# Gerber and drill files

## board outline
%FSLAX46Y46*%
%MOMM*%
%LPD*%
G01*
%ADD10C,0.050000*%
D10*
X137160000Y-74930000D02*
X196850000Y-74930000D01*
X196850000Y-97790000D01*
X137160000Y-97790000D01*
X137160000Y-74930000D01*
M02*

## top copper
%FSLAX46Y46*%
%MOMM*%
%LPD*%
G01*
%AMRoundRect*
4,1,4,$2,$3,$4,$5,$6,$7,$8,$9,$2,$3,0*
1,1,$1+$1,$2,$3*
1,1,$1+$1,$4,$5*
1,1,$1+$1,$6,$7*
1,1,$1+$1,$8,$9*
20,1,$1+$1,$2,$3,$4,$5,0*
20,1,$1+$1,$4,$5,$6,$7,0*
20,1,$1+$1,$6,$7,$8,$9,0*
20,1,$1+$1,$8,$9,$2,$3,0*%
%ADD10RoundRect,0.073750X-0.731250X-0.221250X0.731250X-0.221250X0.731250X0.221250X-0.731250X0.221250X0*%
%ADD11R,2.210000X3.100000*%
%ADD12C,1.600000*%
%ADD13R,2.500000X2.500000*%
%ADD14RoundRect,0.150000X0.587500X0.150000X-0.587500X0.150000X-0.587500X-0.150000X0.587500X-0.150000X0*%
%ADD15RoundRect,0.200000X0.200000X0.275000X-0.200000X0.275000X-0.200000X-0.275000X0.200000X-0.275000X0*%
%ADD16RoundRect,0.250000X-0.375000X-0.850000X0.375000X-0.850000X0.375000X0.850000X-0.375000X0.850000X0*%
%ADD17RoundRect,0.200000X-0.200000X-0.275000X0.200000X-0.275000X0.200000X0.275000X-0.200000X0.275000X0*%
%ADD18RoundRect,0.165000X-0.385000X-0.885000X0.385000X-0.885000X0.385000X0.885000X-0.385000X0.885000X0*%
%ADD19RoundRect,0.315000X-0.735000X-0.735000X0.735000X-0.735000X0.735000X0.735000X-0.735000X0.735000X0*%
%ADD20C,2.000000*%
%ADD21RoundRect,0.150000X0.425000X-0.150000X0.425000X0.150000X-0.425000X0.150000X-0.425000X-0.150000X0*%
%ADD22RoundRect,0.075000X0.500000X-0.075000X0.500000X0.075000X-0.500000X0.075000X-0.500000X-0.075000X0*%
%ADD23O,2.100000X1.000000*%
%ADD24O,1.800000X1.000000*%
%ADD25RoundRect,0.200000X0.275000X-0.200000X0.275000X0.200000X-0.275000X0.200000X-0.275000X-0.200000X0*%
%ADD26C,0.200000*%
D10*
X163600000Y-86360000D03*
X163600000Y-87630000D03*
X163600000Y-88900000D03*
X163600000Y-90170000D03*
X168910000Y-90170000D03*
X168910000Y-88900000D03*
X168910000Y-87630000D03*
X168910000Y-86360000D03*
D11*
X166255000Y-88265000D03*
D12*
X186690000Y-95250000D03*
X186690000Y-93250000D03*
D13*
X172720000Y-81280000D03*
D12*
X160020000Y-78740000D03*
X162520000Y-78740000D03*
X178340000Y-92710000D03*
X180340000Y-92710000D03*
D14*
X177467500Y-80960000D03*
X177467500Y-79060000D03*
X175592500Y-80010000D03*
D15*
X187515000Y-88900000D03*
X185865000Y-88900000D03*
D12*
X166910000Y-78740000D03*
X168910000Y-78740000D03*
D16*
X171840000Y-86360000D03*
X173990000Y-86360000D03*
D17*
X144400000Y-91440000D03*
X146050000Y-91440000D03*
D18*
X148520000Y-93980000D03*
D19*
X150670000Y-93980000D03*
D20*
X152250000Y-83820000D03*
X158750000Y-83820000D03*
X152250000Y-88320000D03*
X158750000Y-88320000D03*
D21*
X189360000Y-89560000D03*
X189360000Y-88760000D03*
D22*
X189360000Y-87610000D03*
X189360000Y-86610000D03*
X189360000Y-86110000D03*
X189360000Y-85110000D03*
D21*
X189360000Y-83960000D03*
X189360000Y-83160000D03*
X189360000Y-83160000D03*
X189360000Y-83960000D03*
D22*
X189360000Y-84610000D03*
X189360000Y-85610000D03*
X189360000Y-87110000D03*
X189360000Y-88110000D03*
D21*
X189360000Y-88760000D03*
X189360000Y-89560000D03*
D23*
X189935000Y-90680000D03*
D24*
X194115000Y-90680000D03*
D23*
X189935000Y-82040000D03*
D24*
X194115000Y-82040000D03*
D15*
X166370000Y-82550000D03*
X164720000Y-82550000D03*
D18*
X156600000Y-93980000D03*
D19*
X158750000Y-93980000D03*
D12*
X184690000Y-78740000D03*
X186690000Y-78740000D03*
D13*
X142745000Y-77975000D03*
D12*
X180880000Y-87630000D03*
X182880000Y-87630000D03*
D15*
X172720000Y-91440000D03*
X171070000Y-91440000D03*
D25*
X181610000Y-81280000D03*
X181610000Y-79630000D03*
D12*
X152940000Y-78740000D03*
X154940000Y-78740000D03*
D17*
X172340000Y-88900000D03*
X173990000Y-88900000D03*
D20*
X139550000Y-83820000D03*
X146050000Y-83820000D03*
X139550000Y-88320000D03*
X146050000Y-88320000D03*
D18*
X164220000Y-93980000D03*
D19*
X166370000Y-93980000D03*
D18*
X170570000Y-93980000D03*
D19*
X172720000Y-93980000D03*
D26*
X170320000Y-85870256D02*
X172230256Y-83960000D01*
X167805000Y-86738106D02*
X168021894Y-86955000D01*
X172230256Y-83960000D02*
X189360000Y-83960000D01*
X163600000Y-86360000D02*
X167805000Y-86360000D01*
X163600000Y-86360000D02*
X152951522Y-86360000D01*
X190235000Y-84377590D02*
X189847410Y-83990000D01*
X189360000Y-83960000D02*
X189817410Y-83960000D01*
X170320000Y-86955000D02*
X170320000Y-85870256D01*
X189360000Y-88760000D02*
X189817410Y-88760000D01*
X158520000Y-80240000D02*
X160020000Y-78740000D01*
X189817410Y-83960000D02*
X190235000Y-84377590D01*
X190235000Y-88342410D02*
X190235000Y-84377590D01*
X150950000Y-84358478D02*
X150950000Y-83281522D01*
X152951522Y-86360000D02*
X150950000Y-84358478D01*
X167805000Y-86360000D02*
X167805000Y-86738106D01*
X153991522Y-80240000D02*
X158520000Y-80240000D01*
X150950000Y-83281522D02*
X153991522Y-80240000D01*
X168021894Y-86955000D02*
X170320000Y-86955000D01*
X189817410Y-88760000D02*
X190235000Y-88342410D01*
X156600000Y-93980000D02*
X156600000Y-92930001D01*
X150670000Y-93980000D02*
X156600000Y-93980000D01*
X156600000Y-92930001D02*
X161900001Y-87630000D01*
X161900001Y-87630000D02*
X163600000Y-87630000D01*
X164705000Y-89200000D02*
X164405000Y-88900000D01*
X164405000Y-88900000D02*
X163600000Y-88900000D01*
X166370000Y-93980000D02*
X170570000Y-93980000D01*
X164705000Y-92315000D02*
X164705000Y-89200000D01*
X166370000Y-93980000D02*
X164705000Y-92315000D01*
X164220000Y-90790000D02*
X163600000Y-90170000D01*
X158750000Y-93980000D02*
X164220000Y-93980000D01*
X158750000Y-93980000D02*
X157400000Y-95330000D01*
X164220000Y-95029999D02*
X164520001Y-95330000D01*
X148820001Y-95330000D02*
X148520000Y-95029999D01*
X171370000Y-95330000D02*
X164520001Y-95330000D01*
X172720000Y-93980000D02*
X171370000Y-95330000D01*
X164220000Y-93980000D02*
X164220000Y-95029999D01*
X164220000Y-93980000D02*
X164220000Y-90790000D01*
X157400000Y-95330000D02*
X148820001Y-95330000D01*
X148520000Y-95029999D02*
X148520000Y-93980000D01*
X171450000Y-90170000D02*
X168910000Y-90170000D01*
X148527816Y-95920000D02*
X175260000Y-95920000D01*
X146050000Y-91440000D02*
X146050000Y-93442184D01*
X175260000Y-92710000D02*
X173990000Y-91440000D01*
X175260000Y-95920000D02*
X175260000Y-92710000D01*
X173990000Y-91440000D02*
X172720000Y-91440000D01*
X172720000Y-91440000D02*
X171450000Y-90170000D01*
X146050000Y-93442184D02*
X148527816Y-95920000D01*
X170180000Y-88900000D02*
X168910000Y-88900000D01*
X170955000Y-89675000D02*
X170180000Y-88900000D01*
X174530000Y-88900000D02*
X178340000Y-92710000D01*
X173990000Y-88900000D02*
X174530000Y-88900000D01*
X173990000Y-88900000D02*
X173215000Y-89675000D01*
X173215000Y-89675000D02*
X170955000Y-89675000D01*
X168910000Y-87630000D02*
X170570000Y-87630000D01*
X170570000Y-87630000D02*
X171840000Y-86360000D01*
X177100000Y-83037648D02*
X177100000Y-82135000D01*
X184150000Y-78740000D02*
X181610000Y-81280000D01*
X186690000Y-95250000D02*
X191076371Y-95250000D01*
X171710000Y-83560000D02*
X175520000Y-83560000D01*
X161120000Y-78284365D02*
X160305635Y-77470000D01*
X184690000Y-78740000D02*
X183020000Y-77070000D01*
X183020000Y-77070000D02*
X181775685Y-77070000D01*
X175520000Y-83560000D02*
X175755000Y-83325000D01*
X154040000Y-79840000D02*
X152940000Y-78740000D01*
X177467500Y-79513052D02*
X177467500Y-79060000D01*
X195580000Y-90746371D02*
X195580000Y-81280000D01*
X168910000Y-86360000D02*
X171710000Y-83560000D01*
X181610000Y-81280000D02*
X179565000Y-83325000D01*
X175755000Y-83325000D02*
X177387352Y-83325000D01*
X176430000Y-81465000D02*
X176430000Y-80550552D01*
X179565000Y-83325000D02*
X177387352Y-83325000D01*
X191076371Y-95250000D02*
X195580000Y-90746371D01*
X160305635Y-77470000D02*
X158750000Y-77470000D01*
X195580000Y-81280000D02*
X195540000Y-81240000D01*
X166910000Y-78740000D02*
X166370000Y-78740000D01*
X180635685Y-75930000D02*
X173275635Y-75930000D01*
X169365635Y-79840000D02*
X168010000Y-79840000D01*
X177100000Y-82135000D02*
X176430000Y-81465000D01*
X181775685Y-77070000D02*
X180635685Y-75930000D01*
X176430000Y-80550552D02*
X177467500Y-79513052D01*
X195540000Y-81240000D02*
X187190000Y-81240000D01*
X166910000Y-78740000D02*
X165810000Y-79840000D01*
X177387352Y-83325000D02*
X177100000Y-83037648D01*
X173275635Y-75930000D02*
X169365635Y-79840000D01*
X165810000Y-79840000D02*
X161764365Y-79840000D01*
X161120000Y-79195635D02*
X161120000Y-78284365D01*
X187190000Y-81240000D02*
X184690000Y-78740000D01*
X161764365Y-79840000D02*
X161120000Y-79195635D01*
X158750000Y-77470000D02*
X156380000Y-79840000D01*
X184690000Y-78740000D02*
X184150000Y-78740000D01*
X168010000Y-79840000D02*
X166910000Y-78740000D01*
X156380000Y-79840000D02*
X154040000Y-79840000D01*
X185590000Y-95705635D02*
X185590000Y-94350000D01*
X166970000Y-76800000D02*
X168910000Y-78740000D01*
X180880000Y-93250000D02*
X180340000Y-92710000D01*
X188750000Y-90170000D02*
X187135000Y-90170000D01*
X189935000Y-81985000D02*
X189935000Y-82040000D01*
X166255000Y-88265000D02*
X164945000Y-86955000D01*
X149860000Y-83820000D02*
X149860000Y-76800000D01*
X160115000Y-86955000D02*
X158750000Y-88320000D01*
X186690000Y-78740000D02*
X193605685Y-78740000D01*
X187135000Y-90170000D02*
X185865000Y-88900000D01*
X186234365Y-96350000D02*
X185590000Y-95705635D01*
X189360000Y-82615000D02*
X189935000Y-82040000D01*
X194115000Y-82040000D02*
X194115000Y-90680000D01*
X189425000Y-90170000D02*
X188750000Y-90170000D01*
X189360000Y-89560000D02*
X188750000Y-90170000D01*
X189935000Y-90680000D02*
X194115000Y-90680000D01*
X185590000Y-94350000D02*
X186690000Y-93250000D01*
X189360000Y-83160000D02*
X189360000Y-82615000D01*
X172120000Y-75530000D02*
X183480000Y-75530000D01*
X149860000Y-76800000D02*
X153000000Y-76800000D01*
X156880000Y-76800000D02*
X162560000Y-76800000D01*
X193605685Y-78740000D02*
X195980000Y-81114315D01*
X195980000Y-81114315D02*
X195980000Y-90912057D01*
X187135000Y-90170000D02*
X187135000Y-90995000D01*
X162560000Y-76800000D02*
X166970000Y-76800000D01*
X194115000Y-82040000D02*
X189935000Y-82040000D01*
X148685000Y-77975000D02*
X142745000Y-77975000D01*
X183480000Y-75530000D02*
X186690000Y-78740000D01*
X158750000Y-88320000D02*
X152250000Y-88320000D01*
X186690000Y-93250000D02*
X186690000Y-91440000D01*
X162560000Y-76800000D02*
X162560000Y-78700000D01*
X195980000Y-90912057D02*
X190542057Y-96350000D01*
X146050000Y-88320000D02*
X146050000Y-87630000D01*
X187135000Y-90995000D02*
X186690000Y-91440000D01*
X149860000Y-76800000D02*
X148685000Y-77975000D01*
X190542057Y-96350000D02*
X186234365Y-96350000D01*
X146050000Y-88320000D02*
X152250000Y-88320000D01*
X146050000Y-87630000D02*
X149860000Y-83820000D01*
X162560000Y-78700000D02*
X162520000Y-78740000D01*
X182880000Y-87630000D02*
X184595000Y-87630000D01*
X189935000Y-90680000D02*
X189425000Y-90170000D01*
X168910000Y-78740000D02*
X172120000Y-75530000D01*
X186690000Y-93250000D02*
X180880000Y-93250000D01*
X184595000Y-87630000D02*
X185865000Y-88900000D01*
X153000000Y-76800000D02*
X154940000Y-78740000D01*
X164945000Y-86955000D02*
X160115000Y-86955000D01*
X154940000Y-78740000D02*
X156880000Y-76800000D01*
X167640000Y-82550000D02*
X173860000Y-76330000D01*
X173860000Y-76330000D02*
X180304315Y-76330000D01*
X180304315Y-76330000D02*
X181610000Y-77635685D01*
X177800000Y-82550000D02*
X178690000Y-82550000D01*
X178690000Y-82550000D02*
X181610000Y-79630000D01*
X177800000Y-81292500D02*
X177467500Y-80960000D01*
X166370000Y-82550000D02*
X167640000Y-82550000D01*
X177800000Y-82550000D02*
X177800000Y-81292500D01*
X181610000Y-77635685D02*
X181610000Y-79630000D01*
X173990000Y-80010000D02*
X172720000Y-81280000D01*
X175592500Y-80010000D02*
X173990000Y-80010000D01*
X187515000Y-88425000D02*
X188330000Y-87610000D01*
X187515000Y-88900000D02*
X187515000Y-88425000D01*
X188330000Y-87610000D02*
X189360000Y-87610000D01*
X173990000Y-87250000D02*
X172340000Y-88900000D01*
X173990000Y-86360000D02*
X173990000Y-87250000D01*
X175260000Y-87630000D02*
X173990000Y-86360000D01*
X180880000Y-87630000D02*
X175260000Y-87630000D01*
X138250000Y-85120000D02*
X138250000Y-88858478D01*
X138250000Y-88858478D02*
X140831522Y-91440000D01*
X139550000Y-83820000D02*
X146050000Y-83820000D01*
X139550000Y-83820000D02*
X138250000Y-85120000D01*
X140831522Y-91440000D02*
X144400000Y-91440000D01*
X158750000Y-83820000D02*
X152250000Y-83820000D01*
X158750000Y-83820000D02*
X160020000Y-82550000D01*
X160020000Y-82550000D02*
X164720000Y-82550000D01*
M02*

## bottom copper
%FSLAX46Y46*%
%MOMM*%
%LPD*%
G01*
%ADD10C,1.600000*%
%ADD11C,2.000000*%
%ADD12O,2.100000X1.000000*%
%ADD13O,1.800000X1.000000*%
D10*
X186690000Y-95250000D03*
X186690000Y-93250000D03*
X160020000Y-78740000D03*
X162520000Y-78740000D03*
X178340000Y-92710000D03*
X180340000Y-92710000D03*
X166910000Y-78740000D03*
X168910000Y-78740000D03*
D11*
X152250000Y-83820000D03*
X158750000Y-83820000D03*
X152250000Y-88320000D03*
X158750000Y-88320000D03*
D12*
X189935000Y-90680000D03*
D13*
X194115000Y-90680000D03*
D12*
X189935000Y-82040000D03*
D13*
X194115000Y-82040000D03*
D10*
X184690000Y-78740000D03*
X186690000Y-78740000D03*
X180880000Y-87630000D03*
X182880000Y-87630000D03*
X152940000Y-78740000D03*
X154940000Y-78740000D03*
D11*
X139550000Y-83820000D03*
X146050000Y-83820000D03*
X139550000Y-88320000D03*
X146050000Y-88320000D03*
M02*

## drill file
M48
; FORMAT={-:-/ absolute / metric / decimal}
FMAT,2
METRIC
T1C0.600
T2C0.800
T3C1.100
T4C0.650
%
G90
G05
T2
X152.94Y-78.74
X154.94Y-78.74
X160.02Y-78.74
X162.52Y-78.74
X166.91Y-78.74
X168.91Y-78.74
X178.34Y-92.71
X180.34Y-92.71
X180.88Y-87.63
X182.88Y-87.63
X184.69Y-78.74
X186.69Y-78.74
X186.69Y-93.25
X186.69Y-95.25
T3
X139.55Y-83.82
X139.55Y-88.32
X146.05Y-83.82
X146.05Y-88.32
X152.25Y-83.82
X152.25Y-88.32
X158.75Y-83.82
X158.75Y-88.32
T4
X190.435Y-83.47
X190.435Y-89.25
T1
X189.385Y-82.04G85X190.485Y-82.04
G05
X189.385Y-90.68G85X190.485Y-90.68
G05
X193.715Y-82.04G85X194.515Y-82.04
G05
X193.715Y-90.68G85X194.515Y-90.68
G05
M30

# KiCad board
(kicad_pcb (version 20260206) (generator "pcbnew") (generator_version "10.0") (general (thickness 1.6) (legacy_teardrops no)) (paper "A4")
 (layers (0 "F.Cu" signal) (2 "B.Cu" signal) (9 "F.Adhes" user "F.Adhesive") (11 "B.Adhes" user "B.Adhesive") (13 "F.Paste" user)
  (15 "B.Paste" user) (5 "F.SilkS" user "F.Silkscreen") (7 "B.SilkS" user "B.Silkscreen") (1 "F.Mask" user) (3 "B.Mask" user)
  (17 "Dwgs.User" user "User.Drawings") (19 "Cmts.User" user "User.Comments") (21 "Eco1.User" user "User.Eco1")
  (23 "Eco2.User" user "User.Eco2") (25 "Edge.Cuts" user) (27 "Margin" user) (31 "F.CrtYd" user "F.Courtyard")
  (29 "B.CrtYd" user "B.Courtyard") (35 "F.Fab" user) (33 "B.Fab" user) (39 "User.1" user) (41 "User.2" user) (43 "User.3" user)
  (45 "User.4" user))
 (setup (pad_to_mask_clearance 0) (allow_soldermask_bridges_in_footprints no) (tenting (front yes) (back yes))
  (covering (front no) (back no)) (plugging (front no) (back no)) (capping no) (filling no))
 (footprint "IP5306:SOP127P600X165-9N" (layer "F.Cu") (at 166.255 88.265)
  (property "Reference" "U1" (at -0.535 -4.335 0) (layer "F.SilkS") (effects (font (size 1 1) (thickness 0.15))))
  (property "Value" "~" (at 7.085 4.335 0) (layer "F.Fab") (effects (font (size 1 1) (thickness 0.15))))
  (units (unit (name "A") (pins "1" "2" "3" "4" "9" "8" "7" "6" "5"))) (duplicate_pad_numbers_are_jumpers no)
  (pad "1" smd roundrect (at -2.655 -1.905) (size 1.61 0.59) (layers "F.Cu" "F.Mask" "F.Paste") (roundrect_rratio 0.125)
   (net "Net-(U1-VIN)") (solder_mask_margin 0.102))
  (pad "2" smd roundrect (at -2.655 -0.635) (size 1.61 0.59) (layers "F.Cu" "F.Mask" "F.Paste") (roundrect_rratio 0.125) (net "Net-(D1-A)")
   (solder_mask_margin 0.102))
  (pad "3" smd roundrect (at -2.655 0.635) (size 1.61 0.59) (layers "F.Cu" "F.Mask" "F.Paste") (roundrect_rratio 0.125) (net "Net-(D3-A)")
   (solder_mask_margin 0.102))
  (pad "4" smd roundrect (at -2.655 1.905) (size 1.61 0.59) (layers "F.Cu" "F.Mask" "F.Paste") (roundrect_rratio 0.125) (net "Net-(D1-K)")
   (solder_mask_margin 0.102))
  (pad "5" smd roundrect (at 2.655 1.905) (size 1.61 0.59) (layers "F.Cu" "F.Mask" "F.Paste") (roundrect_rratio 0.125) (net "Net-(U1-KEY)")
   (solder_mask_margin 0.102))
  (pad "6" smd roundrect (at 2.655 0.635) (size 1.61 0.59) (layers "F.Cu" "F.Mask" "F.Paste") (roundrect_rratio 0.125) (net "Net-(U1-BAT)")
   (solder_mask_margin 0.102))
  (pad "7" smd roundrect (at 2.655 -0.635) (size 1.61 0.59) (layers "F.Cu" "F.Mask" "F.Paste") (roundrect_rratio 0.125) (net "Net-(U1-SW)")
   (solder_mask_margin 0.102))
  (pad "8" smd roundrect (at 2.655 -1.905) (size 1.61 0.59) (layers "F.Cu" "F.Mask" "F.Paste") (roundrect_rratio 0.125) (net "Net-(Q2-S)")
   (solder_mask_margin 0.102))
  (pad "9" smd rect (at 0 0) (size 2.21 3.1) (layers "F.Cu" "F.Mask") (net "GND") (solder_mask_margin 0.102)))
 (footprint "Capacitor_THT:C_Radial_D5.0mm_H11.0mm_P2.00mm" (layer "F.Cu") (at 186.69 95.25 90)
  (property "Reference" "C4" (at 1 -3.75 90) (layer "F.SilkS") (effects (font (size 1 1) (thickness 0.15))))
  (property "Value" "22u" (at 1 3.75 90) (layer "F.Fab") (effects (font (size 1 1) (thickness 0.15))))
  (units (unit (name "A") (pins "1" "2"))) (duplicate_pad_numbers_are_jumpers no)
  (pad "1" thru_hole circle (at 0 0 90) (size 1.6 1.6) (drill 0.8) (layers "*.Cu" "*.Mask") (remove_unused_layers no) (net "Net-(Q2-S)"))
  (pad "2" thru_hole circle (at 2 0 90) (size 1.6 1.6) (drill 0.8) (layers "*.Cu" "*.Mask") (remove_unused_layers no) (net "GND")))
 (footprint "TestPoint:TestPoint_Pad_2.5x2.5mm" (layer "F.Cu") (at 172.72 81.28)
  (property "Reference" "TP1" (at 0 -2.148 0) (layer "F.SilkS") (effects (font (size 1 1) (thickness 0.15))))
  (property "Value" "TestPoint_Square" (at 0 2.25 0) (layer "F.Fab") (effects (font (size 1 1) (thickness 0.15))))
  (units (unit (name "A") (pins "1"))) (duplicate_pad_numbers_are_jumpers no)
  (pad "1" smd rect (at 0 0) (size 2.5 2.5) (layers "F.Cu" "F.Mask") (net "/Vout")))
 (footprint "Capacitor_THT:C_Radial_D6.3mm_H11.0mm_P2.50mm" (layer "F.Cu") (at 160.02 78.74)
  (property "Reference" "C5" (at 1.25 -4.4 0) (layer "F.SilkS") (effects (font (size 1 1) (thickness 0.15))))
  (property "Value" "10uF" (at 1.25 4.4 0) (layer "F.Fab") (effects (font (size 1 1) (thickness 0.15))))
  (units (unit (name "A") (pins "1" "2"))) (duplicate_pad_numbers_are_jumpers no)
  (pad "1" thru_hole circle (at 0 0) (size 1.6 1.6) (drill 0.8) (layers "*.Cu" "*.Mask") (remove_unused_layers no) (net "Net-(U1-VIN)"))
  (pad "2" thru_hole circle (at 2.5 0) (size 1.6 1.6) (drill 0.8) (layers "*.Cu" "*.Mask") (remove_unused_layers no) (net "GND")))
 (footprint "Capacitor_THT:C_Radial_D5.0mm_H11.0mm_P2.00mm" (layer "F.Cu") (at 178.34 92.71)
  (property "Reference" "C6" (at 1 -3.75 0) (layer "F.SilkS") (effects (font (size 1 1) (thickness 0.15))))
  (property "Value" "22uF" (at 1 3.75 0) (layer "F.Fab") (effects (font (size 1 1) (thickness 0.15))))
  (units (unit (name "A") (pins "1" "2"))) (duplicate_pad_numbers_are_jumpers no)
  (pad "1" thru_hole circle (at 0 0) (size 1.6 1.6) (drill 0.8) (layers "*.Cu" "*.Mask") (remove_unused_layers no) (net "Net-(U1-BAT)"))
  (pad "2" thru_hole circle (at 2 0) (size 1.6 1.6) (drill 0.8) (layers "*.Cu" "*.Mask") (remove_unused_layers no) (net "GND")))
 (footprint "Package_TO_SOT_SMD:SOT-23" (layer "F.Cu") (at 176.53 80.01 180)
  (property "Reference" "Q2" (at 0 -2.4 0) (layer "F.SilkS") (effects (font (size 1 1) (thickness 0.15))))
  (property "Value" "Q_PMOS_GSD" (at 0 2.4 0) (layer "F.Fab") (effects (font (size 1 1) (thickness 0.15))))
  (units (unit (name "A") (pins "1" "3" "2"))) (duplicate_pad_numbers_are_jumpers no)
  (pad "1" smd roundrect (at -0.9375 -0.95 180) (size 1.475 0.6) (layers "F.Cu" "F.Mask" "F.Paste") (roundrect_rratio 0.25)
   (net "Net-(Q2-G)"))
  (pad "2" smd roundrect (at -0.9375 0.95 180) (size 1.475 0.6) (layers "F.Cu" "F.Mask" "F.Paste") (roundrect_rratio 0.25)
   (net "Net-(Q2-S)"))
  (pad "3" smd roundrect (at 0.9375 0 180) (size 1.475 0.6) (layers "F.Cu" "F.Mask" "F.Paste") (roundrect_rratio 0.25) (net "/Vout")))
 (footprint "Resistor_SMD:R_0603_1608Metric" (layer "F.Cu") (at 186.69 88.9 180)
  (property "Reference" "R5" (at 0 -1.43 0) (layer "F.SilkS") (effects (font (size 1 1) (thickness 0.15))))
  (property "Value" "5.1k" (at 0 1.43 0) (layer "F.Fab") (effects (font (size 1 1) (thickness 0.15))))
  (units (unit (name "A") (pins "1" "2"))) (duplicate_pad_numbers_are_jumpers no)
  (pad "1" smd roundrect (at -0.825 0 180) (size 0.8 0.95) (layers "F.Cu" "F.Mask" "F.Paste") (roundrect_rratio 0.25) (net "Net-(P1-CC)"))
  (pad "2" smd roundrect (at 0.825 0 180) (size 0.8 0.95) (layers "F.Cu" "F.Mask" "F.Paste") (roundrect_rratio 0.25) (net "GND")))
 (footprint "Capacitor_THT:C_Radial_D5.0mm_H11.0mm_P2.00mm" (layer "F.Cu") (at 166.91 78.74)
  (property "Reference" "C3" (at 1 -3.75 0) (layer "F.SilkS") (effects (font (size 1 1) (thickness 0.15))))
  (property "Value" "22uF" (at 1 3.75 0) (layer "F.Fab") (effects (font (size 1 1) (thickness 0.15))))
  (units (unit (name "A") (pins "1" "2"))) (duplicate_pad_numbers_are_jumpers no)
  (pad "1" thru_hole circle (at 0 0) (size 1.6 1.6) (drill 0.8) (layers "*.Cu" "*.Mask") (remove_unused_layers no) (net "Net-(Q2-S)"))
  (pad "2" thru_hole circle (at 2 0) (size 1.6 1.6) (drill 0.8) (layers "*.Cu" "*.Mask") (remove_unused_layers no) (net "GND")))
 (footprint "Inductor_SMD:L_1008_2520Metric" (layer "F.Cu") (at 172.915 86.36)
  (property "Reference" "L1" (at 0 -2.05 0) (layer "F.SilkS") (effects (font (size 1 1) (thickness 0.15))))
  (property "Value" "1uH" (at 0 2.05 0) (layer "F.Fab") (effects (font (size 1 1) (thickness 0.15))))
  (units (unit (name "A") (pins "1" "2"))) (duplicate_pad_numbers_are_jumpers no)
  (pad "1" smd roundrect (at -1.075 0) (size 1.25 2.2) (layers "F.Cu" "F.Mask" "F.Paste") (roundrect_rratio 0.2) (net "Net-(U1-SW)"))
  (pad "2" smd roundrect (at 1.075 0) (size 1.25 2.2) (layers "F.Cu" "F.Mask" "F.Paste") (roundrect_rratio 0.2) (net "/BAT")))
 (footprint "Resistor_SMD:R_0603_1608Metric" (layer "F.Cu") (at 145.225 91.44)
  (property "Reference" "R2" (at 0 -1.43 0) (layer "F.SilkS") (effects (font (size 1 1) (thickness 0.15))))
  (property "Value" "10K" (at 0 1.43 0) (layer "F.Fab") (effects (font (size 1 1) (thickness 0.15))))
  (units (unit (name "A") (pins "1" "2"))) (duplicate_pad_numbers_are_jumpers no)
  (pad "1" smd roundrect (at -0.825 0) (size 0.8 0.95) (layers "F.Cu" "F.Mask" "F.Paste") (roundrect_rratio 0.25) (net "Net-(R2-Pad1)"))
  (pad "2" smd roundrect (at 0.825 0) (size 0.8 0.95) (layers "F.Cu" "F.Mask" "F.Paste") (roundrect_rratio 0.25) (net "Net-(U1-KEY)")))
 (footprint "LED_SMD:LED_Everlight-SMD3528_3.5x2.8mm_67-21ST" (layer "F.Cu") (at 149.86 93.98)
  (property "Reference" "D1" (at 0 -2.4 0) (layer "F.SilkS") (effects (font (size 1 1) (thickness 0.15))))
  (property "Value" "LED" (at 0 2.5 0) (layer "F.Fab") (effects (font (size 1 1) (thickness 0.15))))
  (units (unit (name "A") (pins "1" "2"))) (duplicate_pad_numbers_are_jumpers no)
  (pad "1" smd roundrect (at -1.34 0) (size 1.1 2.1) (layers "F.Cu" "F.Mask" "F.Paste") (roundrect_rratio 0.15) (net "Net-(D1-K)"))
  (pad "2" smd roundrect (at 0.81 0) (size 2.1 2.1) (layers "F.Cu" "F.Mask" "F.Paste") (roundrect_rratio 0.15) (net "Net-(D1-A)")))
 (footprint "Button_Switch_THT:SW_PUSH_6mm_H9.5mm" (layer "F.Cu") (at 152.25 83.82)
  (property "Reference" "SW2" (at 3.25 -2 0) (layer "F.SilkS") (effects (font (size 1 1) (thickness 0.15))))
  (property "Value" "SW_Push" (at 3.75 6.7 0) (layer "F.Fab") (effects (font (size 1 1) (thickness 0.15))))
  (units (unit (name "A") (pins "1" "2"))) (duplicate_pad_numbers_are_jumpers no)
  (pad "1" thru_hole circle (at 0 0 90) (size 2 2) (drill 1.1) (layers "*.Cu" "*.Mask") (remove_unused_layers no) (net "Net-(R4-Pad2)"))
  (pad "1" thru_hole circle (at 6.5 0 90) (size 2 2) (drill 1.1) (layers "*.Cu" "*.Mask") (remove_unused_layers no) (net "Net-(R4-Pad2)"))
  (pad "2" thru_hole circle (at 0 4.5 90) (size 2 2) (drill 1.1) (layers "*.Cu" "*.Mask") (remove_unused_layers no) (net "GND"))
  (pad "2" thru_hole circle (at 6.5 4.5 90) (size 2 2) (drill 1.1) (layers "*.Cu" "*.Mask") (remove_unused_layers no) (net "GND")))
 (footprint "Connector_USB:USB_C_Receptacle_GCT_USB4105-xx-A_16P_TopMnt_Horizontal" (layer "F.Cu") (at 193.04 86.36 90)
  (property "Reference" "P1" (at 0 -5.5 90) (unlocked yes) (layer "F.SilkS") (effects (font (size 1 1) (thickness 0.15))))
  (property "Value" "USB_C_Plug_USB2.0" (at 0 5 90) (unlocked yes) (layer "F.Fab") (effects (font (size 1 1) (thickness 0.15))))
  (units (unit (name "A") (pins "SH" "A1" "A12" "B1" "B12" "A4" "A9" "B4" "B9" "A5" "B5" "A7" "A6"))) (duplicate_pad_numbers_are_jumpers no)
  (pad "" np_thru_hole circle (at -2.89 -2.605 90) (size 0.65 0.65) (drill 0.65) (layers "*.Cu" "*.Mask"))
  (pad "" np_thru_hole circle (at 2.89 -2.605 90) (size 0.65 0.65) (drill 0.65) (layers "*.Cu" "*.Mask"))
  (pad "A1" smd roundrect (at -3.2 -3.68 90) (size 0.6 1.15) (layers "F.Cu" "F.Mask" "F.Paste") (roundrect_rratio 0.25) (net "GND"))
  (pad "A4" smd roundrect (at -2.4 -3.68 90) (size 0.6 1.15) (layers "F.Cu" "F.Mask" "F.Paste") (roundrect_rratio 0.25) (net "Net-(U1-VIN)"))
  (pad "A5" smd roundrect (at -1.25 -3.68 90) (size 0.3 1.15) (layers "F.Cu" "F.Mask" "F.Paste") (roundrect_rratio 0.25) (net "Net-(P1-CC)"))
  (pad "A6" smd roundrect (at -0.25 -3.68 90) (size 0.3 1.15) (layers "F.Cu" "F.Mask" "F.Paste") (roundrect_rratio 0.25)
   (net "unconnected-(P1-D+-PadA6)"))
  (pad "A7" smd roundrect (at 0.25 -3.68 90) (size 0.3 1.15) (layers "F.Cu" "F.Mask" "F.Paste") (roundrect_rratio 0.25)
   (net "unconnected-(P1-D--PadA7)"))
  (pad "A8" smd roundrect (at 1.25 -3.68 90) (size 0.3 1.15) (layers "F.Cu" "F.Mask" "F.Paste") (roundrect_rratio 0.25))
  (pad "A9" smd roundrect (at 2.4 -3.68 90) (size 0.6 1.15) (layers "F.Cu" "F.Mask" "F.Paste") (roundrect_rratio 0.25) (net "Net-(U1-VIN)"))
  (pad "A12" smd roundrect (at 3.2 -3.68 90) (size 0.6 1.15) (layers "F.Cu" "F.Mask" "F.Paste") (roundrect_rratio 0.25) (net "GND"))
  (pad "B1" smd roundrect (at 3.2 -3.68 90) (size 0.6 1.15) (layers "F.Cu" "F.Mask" "F.Paste") (roundrect_rratio 0.25) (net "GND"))
  (pad "B4" smd roundrect (at 2.4 -3.68 90) (size 0.6 1.15) (layers "F.Cu" "F.Mask" "F.Paste") (roundrect_rratio 0.25) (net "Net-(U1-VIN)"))
  (pad "B5" smd roundrect (at 1.75 -3.68 90) (size 0.3 1.15) (layers "F.Cu" "F.Mask" "F.Paste") (roundrect_rratio 0.25)
   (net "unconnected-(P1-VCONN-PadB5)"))
  (pad "B6" smd roundrect (at 0.75 -3.68 90) (size 0.3 1.15) (layers "F.Cu" "F.Mask" "F.Paste") (roundrect_rratio 0.25))
  (pad "B7" smd roundrect (at -0.75 -3.68 90) (size 0.3 1.15) (layers "F.Cu" "F.Mask" "F.Paste") (roundrect_rratio 0.25))
  (pad "B8" smd roundrect (at -1.75 -3.68 90) (size 0.3 1.15) (layers "F.Cu" "F.Mask" "F.Paste") (roundrect_rratio 0.25))
  (pad "B9" smd roundrect (at -2.4 -3.68 90) (size 0.6 1.15) (layers "F.Cu" "F.Mask" "F.Paste") (roundrect_rratio 0.25) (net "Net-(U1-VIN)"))
  (pad "B12" smd roundrect (at -3.2 -3.68 90) (size 0.6 1.15) (layers "F.Cu" "F.Mask" "F.Paste") (roundrect_rratio 0.25) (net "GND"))
  (pad "SH" thru_hole oval (at -4.32 -3.105 90) (size 1 2.1) (drill oval 0.6 1.7) (layers "*.Cu" "*.Mask" "F.Paste")
   (remove_unused_layers no) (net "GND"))
  (pad "SH" thru_hole oval (at -4.32 1.075 90) (size 1 1.8) (drill oval 0.6 1.4) (layers "*.Cu" "*.Mask" "F.Paste")
   (remove_unused_layers no) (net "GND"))
  (pad "SH" thru_hole oval (at 4.32 -3.105 90) (size 1 2.1) (drill oval 0.6 1.7) (layers "*.Cu" "*.Mask" "F.Paste")
   (remove_unused_layers no) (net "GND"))
  (pad "SH" thru_hole oval (at 4.32 1.075 90) (size 1 1.8) (drill oval 0.6 1.4) (layers "*.Cu" "*.Mask" "F.Paste") (remove_unused_layers no)
   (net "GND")))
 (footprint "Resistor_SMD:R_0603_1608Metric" (layer "F.Cu") (at 165.545 82.55 180)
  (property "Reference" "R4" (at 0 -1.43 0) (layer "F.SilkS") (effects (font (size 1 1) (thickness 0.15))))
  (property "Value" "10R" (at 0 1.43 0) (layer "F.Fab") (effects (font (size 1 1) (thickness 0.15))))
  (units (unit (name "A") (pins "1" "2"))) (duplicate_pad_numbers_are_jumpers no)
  (pad "1" smd roundrect (at -0.825 0 180) (size 0.8 0.95) (layers "F.Cu" "F.Mask" "F.Paste") (roundrect_rratio 0.25) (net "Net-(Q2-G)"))
  (pad "2" smd roundrect (at 0.825 0 180) (size 0.8 0.95) (layers "F.Cu" "F.Mask" "F.Paste") (roundrect_rratio 0.25) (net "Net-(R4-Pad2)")))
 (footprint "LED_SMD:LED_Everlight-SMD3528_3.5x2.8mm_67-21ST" (layer "F.Cu") (at 157.94 93.98)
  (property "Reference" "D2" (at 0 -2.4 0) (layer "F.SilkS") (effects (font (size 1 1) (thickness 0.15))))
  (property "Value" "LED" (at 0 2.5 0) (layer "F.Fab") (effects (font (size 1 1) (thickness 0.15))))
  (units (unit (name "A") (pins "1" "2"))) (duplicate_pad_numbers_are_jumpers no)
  (pad "1" smd roundrect (at -1.34 0) (size 1.1 2.1) (layers "F.Cu" "F.Mask" "F.Paste") (roundrect_rratio 0.15) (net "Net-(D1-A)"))
  (pad "2" smd roundrect (at 0.81 0) (size 2.1 2.1) (layers "F.Cu" "F.Mask" "F.Paste") (roundrect_rratio 0.15) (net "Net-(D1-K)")))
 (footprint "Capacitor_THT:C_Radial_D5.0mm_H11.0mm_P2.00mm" (layer "F.Cu") (at 184.69 78.74)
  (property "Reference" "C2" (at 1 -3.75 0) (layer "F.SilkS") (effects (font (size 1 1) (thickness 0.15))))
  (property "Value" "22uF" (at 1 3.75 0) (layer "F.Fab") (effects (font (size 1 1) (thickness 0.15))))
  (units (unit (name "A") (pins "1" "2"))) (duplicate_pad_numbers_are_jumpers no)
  (pad "1" thru_hole circle (at 0 0) (size 1.6 1.6) (drill 0.8) (layers "*.Cu" "*.Mask") (remove_unused_layers no) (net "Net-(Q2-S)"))
  (pad "2" thru_hole circle (at 2 0) (size 1.6 1.6) (drill 0.8) (layers "*.Cu" "*.Mask") (remove_unused_layers no) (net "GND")))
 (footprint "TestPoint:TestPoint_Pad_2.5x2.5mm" (layer "F.Cu") (at 142.745 77.975)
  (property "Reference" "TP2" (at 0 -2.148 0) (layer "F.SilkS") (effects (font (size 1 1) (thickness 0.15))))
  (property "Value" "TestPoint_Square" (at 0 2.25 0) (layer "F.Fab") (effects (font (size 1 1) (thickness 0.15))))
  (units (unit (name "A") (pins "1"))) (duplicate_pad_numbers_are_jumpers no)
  (pad "1" smd rect (at 0 0) (size 2.5 2.5) (layers "F.Cu" "F.Mask") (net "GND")))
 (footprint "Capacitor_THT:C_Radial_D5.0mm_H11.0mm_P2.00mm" (layer "F.Cu") (at 180.88 87.63)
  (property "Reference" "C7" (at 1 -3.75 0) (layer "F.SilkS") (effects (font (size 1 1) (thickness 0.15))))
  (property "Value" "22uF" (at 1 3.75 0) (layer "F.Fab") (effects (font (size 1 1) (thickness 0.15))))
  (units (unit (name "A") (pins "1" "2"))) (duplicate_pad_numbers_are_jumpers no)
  (pad "1" thru_hole circle (at 0 0) (size 1.6 1.6) (drill 0.8) (layers "*.Cu" "*.Mask") (remove_unused_layers no) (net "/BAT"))
  (pad "2" thru_hole circle (at 2 0) (size 1.6 1.6) (drill 0.8) (layers "*.Cu" "*.Mask") (remove_unused_layers no) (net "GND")))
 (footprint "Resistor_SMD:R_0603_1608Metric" (layer "F.Cu") (at 171.895 91.44 180)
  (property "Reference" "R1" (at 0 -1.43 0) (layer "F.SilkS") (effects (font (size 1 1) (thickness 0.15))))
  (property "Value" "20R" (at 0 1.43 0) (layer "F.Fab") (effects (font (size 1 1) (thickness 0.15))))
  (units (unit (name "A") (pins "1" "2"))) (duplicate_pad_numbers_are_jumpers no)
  (pad "1" smd roundrect (at -0.825 0 180) (size 0.8 0.95) (layers "F.Cu" "F.Mask" "F.Paste") (roundrect_rratio 0.25) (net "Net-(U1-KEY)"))
  (pad "2" smd roundrect (at 0.825 0 180) (size 0.8 0.95) (layers "F.Cu" "F.Mask" "F.Paste") (roundrect_rratio 0.25) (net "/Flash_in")))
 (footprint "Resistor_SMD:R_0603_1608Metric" (layer "F.Cu") (at 181.61 80.455 90)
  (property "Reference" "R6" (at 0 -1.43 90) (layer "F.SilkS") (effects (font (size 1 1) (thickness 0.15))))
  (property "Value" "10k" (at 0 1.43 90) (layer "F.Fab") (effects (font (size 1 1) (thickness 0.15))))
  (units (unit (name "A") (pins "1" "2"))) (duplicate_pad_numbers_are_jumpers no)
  (pad "1" smd roundrect (at -0.825 0 90) (size 0.8 0.95) (layers "F.Cu" "F.Mask" "F.Paste") (roundrect_rratio 0.25) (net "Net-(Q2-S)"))
  (pad "2" smd roundrect (at 0.825 0 90) (size 0.8 0.95) (layers "F.Cu" "F.Mask" "F.Paste") (roundrect_rratio 0.25) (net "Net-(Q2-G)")))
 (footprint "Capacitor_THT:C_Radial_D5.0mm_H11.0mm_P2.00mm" (layer "F.Cu") (at 152.94 78.74)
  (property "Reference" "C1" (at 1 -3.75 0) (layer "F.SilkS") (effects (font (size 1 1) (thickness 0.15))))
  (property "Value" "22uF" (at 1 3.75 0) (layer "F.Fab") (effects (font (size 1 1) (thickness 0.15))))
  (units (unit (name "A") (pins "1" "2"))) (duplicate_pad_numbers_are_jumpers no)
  (pad "1" thru_hole circle (at 0 0) (size 1.6 1.6) (drill 0.8) (layers "*.Cu" "*.Mask") (remove_unused_layers no) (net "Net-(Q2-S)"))
  (pad "2" thru_hole circle (at 2 0) (size 1.6 1.6) (drill 0.8) (layers "*.Cu" "*.Mask") (remove_unused_layers no) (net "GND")))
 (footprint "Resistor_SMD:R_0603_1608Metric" (layer "F.Cu") (at 173.165 88.9)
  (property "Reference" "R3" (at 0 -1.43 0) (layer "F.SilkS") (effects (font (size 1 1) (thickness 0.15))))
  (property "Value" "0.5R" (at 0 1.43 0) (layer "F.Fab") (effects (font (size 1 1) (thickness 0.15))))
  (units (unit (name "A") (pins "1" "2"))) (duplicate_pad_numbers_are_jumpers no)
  (pad "1" smd roundrect (at -0.825 0) (size 0.8 0.95) (layers "F.Cu" "F.Mask" "F.Paste") (roundrect_rratio 0.25) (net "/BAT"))
  (pad "2" smd roundrect (at 0.825 0) (size 0.8 0.95) (layers "F.Cu" "F.Mask" "F.Paste") (roundrect_rratio 0.25) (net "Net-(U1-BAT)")))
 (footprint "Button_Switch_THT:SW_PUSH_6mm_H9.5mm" (layer "F.Cu") (at 139.55 83.82)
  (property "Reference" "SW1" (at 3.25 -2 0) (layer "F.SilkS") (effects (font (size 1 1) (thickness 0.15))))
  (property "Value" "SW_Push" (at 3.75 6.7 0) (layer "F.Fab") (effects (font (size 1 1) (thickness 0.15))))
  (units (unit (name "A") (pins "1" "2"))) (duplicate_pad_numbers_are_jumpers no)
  (pad "1" thru_hole circle (at 0 0 90) (size 2 2) (drill 1.1) (layers "*.Cu" "*.Mask") (remove_unused_layers no) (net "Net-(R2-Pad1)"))
  (pad "1" thru_hole circle (at 6.5 0 90) (size 2 2) (drill 1.1) (layers "*.Cu" "*.Mask") (remove_unused_layers no) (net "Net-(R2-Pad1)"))
  (pad "2" thru_hole circle (at 0 4.5 90) (size 2 2) (drill 1.1) (layers "*.Cu" "*.Mask") (remove_unused_layers no) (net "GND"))
  (pad "2" thru_hole circle (at 6.5 4.5 90) (size 2 2) (drill 1.1) (layers "*.Cu" "*.Mask") (remove_unused_layers no) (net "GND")))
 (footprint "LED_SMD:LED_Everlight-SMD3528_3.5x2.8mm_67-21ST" (layer "F.Cu") (at 165.56 93.98)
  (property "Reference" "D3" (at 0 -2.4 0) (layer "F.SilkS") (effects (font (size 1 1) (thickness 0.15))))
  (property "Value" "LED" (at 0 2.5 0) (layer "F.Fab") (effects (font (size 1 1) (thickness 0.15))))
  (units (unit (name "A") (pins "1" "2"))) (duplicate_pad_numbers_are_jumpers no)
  (pad "1" smd roundrect (at -1.34 0) (size 1.1 2.1) (layers "F.Cu" "F.Mask" "F.Paste") (roundrect_rratio 0.15) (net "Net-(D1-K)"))
  (pad "2" smd roundrect (at 0.81 0) (size 2.1 2.1) (layers "F.Cu" "F.Mask" "F.Paste") (roundrect_rratio 0.15) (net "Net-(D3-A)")))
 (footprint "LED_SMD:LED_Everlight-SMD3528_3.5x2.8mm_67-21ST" (layer "F.Cu") (at 171.91 93.98)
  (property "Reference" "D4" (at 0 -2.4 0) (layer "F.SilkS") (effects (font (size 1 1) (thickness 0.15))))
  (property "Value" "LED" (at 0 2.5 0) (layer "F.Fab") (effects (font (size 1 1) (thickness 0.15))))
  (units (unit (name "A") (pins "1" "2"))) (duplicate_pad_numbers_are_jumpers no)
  (pad "1" smd roundrect (at -1.34 0) (size 1.1 2.1) (layers "F.Cu" "F.Mask" "F.Paste") (roundrect_rratio 0.15) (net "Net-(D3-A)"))
  (pad "2" smd roundrect (at 0.81 0) (size 2.1 2.1) (layers "F.Cu" "F.Mask" "F.Paste") (roundrect_rratio 0.15) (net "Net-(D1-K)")))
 (gr_rect (start 137.16 74.93) (end 196.85 97.79) (stroke (width 0.05) (type default)) (fill no) (layer "Edge.Cuts"))
 (segment (start 170.32 85.870256) (end 172.230256 83.96) (width 0.2) (layer "F.Cu") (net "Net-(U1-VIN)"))
 (segment (start 167.805 86.738106) (end 168.021894 86.955) (width 0.2) (layer "F.Cu") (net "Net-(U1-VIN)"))
 (segment (start 172.230256 83.96) (end 189.36 83.96) (width 0.2) (layer "F.Cu") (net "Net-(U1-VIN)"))
 (segment (start 163.6 86.36) (end 167.805 86.36) (width 0.2) (layer "F.Cu") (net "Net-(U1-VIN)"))
 (segment (start 163.6 86.36) (end 152.951522 86.36) (width 0.2) (layer "F.Cu") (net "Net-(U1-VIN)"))
 (segment (start 190.235 84.37759) (end 189.84741 83.99) (width 0.2) (layer "F.Cu") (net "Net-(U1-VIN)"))
 (segment (start 189.36 83.96) (end 189.81741 83.96) (width 0.2) (layer "F.Cu") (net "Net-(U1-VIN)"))
 (segment (start 170.32 86.955) (end 170.32 85.870256) (width 0.2) (layer "F.Cu") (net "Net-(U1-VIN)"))
 (segment (start 189.36 88.76) (end 189.81741 88.76) (width 0.2) (layer "F.Cu") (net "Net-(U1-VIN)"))
 (segment (start 158.52 80.24) (end 160.02 78.74) (width 0.2) (layer "F.Cu") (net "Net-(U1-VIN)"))
 (segment (start 189.81741 83.96) (end 190.235 84.37759) (width 0.2) (layer "F.Cu") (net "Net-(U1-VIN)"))
 (segment (start 190.235 88.34241) (end 190.235 84.37759) (width 0.2) (layer "F.Cu") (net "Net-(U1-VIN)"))
 (segment (start 150.95 84.358478) (end 150.95 83.281522) (width 0.2) (layer "F.Cu") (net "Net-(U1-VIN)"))
 (segment (start 152.951522 86.36) (end 150.95 84.358478) (width 0.2) (layer "F.Cu") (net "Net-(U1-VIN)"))
 (segment (start 167.805 86.36) (end 167.805 86.738106) (width 0.2) (layer "F.Cu") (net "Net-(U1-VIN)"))
 (segment (start 153.991522 80.24) (end 158.52 80.24) (width 0.2) (layer "F.Cu") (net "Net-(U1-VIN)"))
 (segment (start 150.95 83.281522) (end 153.991522 80.24) (width 0.2) (layer "F.Cu") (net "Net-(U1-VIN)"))
 (segment (start 168.021894 86.955) (end 170.32 86.955) (width 0.2) (layer "F.Cu") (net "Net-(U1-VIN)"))
 (segment (start 189.81741 88.76) (end 190.235 88.34241) (width 0.2) (layer "F.Cu") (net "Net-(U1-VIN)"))
 (segment (start 156.6 93.98) (end 156.6 92.930001) (width 0.2) (layer "F.Cu") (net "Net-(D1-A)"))
 (segment (start 150.67 93.98) (end 156.6 93.98) (width 0.2) (layer "F.Cu") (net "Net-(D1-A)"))
 (segment (start 156.6 92.930001) (end 161.900001 87.63) (width 0.2) (layer "F.Cu") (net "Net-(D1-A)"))
 (segment (start 161.900001 87.63) (end 163.6 87.63) (width 0.2) (layer "F.Cu") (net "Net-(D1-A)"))
 (segment (start 164.705 89.2) (end 164.405 88.9) (width 0.2) (layer "F.Cu") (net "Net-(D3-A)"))
 (segment (start 164.405 88.9) (end 163.6 88.9) (width 0.2) (layer "F.Cu") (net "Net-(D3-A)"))
 (segment (start 166.37 93.98) (end 170.57 93.98) (width 0.2) (layer "F.Cu") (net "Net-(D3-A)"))
 (segment (start 164.705 92.315) (end 164.705 89.2) (width 0.2) (layer "F.Cu") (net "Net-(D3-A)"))
 (segment (start 166.37 93.98) (end 164.705 92.315) (width 0.2) (layer "F.Cu") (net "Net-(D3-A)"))
 (segment (start 164.22 90.79) (end 163.6 90.17) (width 0.2) (layer "F.Cu") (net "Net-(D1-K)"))
 (segment (start 158.75 93.98) (end 164.22 93.98) (width 0.2) (layer "F.Cu") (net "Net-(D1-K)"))
 (segment (start 158.75 93.98) (end 157.4 95.33) (width 0.2) (layer "F.Cu") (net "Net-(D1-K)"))
 (segment (start 164.22 95.029999) (end 164.520001 95.33) (width 0.2) (layer "F.Cu") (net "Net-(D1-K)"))
 (segment (start 148.820001 95.33) (end 148.52 95.029999) (width 0.2) (layer "F.Cu") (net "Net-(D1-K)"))
 (segment (start 171.37 95.33) (end 164.520001 95.33) (width 0.2) (layer "F.Cu") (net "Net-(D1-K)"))
 (segment (start 172.72 93.98) (end 171.37 95.33) (width 0.2) (layer "F.Cu") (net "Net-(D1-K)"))
 (segment (start 164.22 93.98) (end 164.22 95.029999) (width 0.2) (layer "F.Cu") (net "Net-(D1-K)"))
 (segment (start 164.22 93.98) (end 164.22 90.79) (width 0.2) (layer "F.Cu") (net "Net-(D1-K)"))
 (segment (start 157.4 95.33) (end 148.820001 95.33) (width 0.2) (layer "F.Cu") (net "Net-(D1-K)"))
 (segment (start 148.52 95.029999) (end 148.52 93.98) (width 0.2) (layer "F.Cu") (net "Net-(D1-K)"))
 (segment (start 171.45 90.17) (end 168.91 90.17) (width 0.2) (layer "F.Cu") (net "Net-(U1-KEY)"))
 (segment (start 148.527816 95.92) (end 175.26 95.92) (width 0.2) (layer "F.Cu") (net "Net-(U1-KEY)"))
 (segment (start 146.05 91.44) (end 146.05 93.442184) (width 0.2) (layer "F.Cu") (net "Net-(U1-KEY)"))
 (segment (start 175.26 92.71) (end 173.99 91.44) (width 0.2) (layer "F.Cu") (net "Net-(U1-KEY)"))
 (segment (start 175.26 95.92) (end 175.26 92.71) (width 0.2) (layer "F.Cu") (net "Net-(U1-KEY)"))
 (segment (start 173.99 91.44) (end 172.72 91.44) (width 0.2) (layer "F.Cu") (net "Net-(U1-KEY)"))
 (segment (start 172.72 91.44) (end 171.45 90.17) (width 0.2) (layer "F.Cu") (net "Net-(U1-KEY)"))
 (segment (start 146.05 93.442184) (end 148.527816 95.92) (width 0.2) (layer "F.Cu") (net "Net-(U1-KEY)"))
 (segment (start 170.18 88.9) (end 168.91 88.9) (width 0.2) (layer "F.Cu") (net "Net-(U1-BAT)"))
 (segment (start 170.955 89.675) (end 170.18 88.9) (width 0.2) (layer "F.Cu") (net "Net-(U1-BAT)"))
 (segment (start 174.53 88.9) (end 178.34 92.71) (width 0.2) (layer "F.Cu") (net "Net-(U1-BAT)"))
 (segment (start 173.99 88.9) (end 174.53 88.9) (width 0.2) (layer "F.Cu") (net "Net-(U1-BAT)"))
 (segment (start 173.99 88.9) (end 173.215 89.675) (width 0.2) (layer "F.Cu") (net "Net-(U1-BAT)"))
 (segment (start 173.215 89.675) (end 170.955 89.675) (width 0.2) (layer "F.Cu") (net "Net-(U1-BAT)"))
 (segment (start 168.91 87.63) (end 170.57 87.63) (width 0.2) (layer "F.Cu") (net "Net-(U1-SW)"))
 (segment (start 170.57 87.63) (end 171.84 86.36) (width 0.2) (layer "F.Cu") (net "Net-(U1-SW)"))
 (segment (start 177.1 83.037648) (end 177.1 82.135) (width 0.2) (layer "F.Cu") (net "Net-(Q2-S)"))
 (segment (start 184.15 78.74) (end 181.61 81.28) (width 0.2) (layer "F.Cu") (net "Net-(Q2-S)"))
 (segment (start 186.69 95.25) (end 191.076371 95.25) (width 0.2) (layer "F.Cu") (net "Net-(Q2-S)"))
 (segment (start 171.71 83.56) (end 175.52 83.56) (width 0.2) (layer "F.Cu") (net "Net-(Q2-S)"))
 (segment (start 161.12 78.284365) (end 160.305635 77.47) (width 0.2) (layer "F.Cu") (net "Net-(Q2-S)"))
 (segment (start 184.69 78.74) (end 183.02 77.07) (width 0.2) (layer "F.Cu") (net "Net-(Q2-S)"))
 (segment (start 183.02 77.07) (end 181.775685 77.07) (width 0.2) (layer "F.Cu") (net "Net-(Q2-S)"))
 (segment (start 175.52 83.56) (end 175.755 83.325) (width 0.2) (layer "F.Cu") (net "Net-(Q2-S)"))
 (segment (start 154.04 79.84) (end 152.94 78.74) (width 0.2) (layer "F.Cu") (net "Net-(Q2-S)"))
 (segment (start 177.4675 79.513052) (end 177.4675 79.06) (width 0.2) (layer "F.Cu") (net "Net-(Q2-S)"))
 (segment (start 195.58 90.746371) (end 195.58 81.28) (width 0.2) (layer "F.Cu") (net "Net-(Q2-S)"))
 (segment (start 168.91 86.36) (end 171.71 83.56) (width 0.2) (layer "F.Cu") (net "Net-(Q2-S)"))
 (segment (start 181.61 81.28) (end 179.565 83.325) (width 0.2) (layer "F.Cu") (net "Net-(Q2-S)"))
 (segment (start 175.755 83.325) (end 177.387352 83.325) (width 0.2) (layer "F.Cu") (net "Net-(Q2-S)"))
 (segment (start 176.43 81.465) (end 176.43 80.550552) (width 0.2) (layer "F.Cu") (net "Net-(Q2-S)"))
 (segment (start 179.565 83.325) (end 177.387352 83.325) (width 0.2) (layer "F.Cu") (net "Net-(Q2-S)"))
 (segment (start 191.076371 95.25) (end 195.58 90.746371) (width 0.2) (layer "F.Cu") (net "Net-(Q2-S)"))
 (segment (start 160.305635 77.47) (end 158.75 77.47) (width 0.2) (layer "F.Cu") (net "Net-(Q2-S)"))
 (segment (start 195.58 81.28) (end 195.54 81.24) (width 0.2) (layer "F.Cu") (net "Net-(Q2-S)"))
 (segment (start 166.91 78.74) (end 166.37 78.74) (width 0.2) (layer "F.Cu") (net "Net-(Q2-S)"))
 (segment (start 180.635685 75.93) (end 173.275635 75.93) (width 0.2) (layer "F.Cu") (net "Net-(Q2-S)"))
 (segment (start 169.365635 79.84) (end 168.01 79.84) (width 0.2) (layer "F.Cu") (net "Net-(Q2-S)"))
 (segment (start 177.1 82.135) (end 176.43 81.465) (width 0.2) (layer "F.Cu") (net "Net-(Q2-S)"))
 (segment (start 181.775685 77.07) (end 180.635685 75.93) (width 0.2) (layer "F.Cu") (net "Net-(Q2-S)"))
 (segment (start 176.43 80.550552) (end 177.4675 79.513052) (width 0.2) (layer "F.Cu") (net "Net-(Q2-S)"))
 (segment (start 195.54 81.24) (end 187.19 81.24) (width 0.2) (layer "F.Cu") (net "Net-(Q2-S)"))
 (segment (start 166.91 78.74) (end 165.81 79.84) (width 0.2) (layer "F.Cu") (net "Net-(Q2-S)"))
 (segment (start 177.387352 83.325) (end 177.1 83.037648) (width 0.2) (layer "F.Cu") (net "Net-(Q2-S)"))
 (segment (start 173.275635 75.93) (end 169.365635 79.84) (width 0.2) (layer "F.Cu") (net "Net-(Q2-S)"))
 (segment (start 165.81 79.84) (end 161.764365 79.84) (width 0.2) (layer "F.Cu") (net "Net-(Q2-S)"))
 (segment (start 161.12 79.195635) (end 161.12 78.284365) (width 0.2) (layer "F.Cu") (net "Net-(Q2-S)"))
 (segment (start 187.19 81.24) (end 184.69 78.74) (width 0.2) (layer "F.Cu") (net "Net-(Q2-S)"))
 (segment (start 161.764365 79.84) (end 161.12 79.195635) (width 0.2) (layer "F.Cu") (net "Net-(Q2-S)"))
 (segment (start 158.75 77.47) (end 156.38 79.84) (width 0.2) (layer "F.Cu") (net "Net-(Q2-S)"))
 (segment (start 184.69 78.74) (end 184.15 78.74) (width 0.2) (layer "F.Cu") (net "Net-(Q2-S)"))
 (segment (start 168.01 79.84) (end 166.91 78.74) (width 0.2) (layer "F.Cu") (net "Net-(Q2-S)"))
 (segment (start 156.38 79.84) (end 154.04 79.84) (width 0.2) (layer "F.Cu") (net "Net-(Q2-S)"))
 (segment (start 185.59 95.705635) (end 185.59 94.35) (width 0.2) (layer "F.Cu") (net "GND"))
 (segment (start 166.97 76.8) (end 168.91 78.74) (width 0.2) (layer "F.Cu") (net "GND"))
 (segment (start 180.88 93.25) (end 180.34 92.71) (width 0.2) (layer "F.Cu") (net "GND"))
 (segment (start 188.75 90.17) (end 187.135 90.17) (width 0.2) (layer "F.Cu") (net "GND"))
 (segment (start 189.935 81.985) (end 189.935 82.04) (width 0.2) (layer "F.Cu") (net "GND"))
 (segment (start 166.255 88.265) (end 164.945 86.955) (width 0.2) (layer "F.Cu") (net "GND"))
 (segment (start 149.86 83.82) (end 149.86 76.8) (width 0.2) (layer "F.Cu") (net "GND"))
 (segment (start 160.115 86.955) (end 158.75 88.32) (width 0.2) (layer "F.Cu") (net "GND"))
 (segment (start 186.69 78.74) (end 193.605685 78.74) (width 0.2) (layer "F.Cu") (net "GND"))
 (segment (start 187.135 90.17) (end 185.865 88.9) (width 0.2) (layer "F.Cu") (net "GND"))
 (segment (start 186.234365 96.35) (end 185.59 95.705635) (width 0.2) (layer "F.Cu") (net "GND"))
 (segment (start 189.36 82.615) (end 189.935 82.04) (width 0.2) (layer "F.Cu") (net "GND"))
 (segment (start 194.115 82.04) (end 194.115 90.68) (width 0.2) (layer "F.Cu") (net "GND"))
 (segment (start 189.425 90.17) (end 188.75 90.17) (width 0.2) (layer "F.Cu") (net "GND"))
 (segment (start 189.36 89.56) (end 188.75 90.17) (width 0.2) (layer "F.Cu") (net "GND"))
 (segment (start 189.935 90.68) (end 194.115 90.68) (width 0.2) (layer "F.Cu") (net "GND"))
 (segment (start 185.59 94.35) (end 186.69 93.25) (width 0.2) (layer "F.Cu") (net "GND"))
 (segment (start 189.36 83.16) (end 189.36 82.615) (width 0.2) (layer "F.Cu") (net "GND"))
 (segment (start 172.12 75.53) (end 183.48 75.53) (width 0.2) (layer "F.Cu") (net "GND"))
 (segment (start 149.86 76.8) (end 153 76.8) (width 0.2) (layer "F.Cu") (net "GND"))
 (segment (start 156.88 76.8) (end 162.56 76.8) (width 0.2) (layer "F.Cu") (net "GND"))
 (segment (start 193.605685 78.74) (end 195.98 81.114315) (width 0.2) (layer "F.Cu") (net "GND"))
 (segment (start 195.98 81.114315) (end 195.98 90.912057) (width 0.2) (layer "F.Cu") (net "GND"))
 (segment (start 187.135 90.17) (end 187.135 90.995) (width 0.2) (layer "F.Cu") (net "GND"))
 (segment (start 162.56 76.8) (end 166.97 76.8) (width 0.2) (layer "F.Cu") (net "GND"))
 (segment (start 194.115 82.04) (end 189.935 82.04) (width 0.2) (layer "F.Cu") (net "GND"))
 (segment (start 148.685 77.975) (end 142.745 77.975) (width 0.2) (layer "F.Cu") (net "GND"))
 (segment (start 183.48 75.53) (end 186.69 78.74) (width 0.2) (layer "F.Cu") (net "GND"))
 (segment (start 158.75 88.32) (end 152.25 88.32) (width 0.2) (layer "F.Cu") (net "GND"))
 (segment (start 186.69 93.25) (end 186.69 91.44) (width 0.2) (layer "F.Cu") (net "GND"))
 (segment (start 162.56 76.8) (end 162.56 78.7) (width 0.2) (layer "F.Cu") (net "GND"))
 (segment (start 195.98 90.912057) (end 190.542057 96.35) (width 0.2) (layer "F.Cu") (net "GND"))
 (segment (start 146.05 88.32) (end 146.05 87.63) (width 0.2) (layer "F.Cu") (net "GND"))
 (segment (start 187.135 90.995) (end 186.69 91.44) (width 0.2) (layer "F.Cu") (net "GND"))
 (segment (start 149.86 76.8) (end 148.685 77.975) (width 0.2) (layer "F.Cu") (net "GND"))
 (segment (start 190.542057 96.35) (end 186.234365 96.35) (width 0.2) (layer "F.Cu") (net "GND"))
 (segment (start 146.05 88.32) (end 152.25 88.32) (width 0.2) (layer "F.Cu") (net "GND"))
 (segment (start 146.05 87.63) (end 149.86 83.82) (width 0.2) (layer "F.Cu") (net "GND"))
 (segment (start 162.56 78.7) (end 162.52 78.74) (width 0.2) (layer "F.Cu") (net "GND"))
 (segment (start 182.88 87.63) (end 184.595 87.63) (width 0.2) (layer "F.Cu") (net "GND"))
 (segment (start 189.935 90.68) (end 189.425 90.17) (width 0.2) (layer "F.Cu") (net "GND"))
 (segment (start 168.91 78.74) (end 172.12 75.53) (width 0.2) (layer "F.Cu") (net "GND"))
 (segment (start 186.69 93.25) (end 180.88 93.25) (width 0.2) (layer "F.Cu") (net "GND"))
 (segment (start 184.595 87.63) (end 185.865 88.9) (width 0.2) (layer "F.Cu") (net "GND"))
 (segment (start 153 76.8) (end 154.94 78.74) (width 0.2) (layer "F.Cu") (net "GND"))
 (segment (start 164.945 86.955) (end 160.115 86.955) (width 0.2) (layer "F.Cu") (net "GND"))
 (segment (start 154.94 78.74) (end 156.88 76.8) (width 0.2) (layer "F.Cu") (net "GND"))
 (segment (start 167.64 82.55) (end 173.86 76.33) (width 0.2) (layer "F.Cu") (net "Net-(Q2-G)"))
 (segment (start 173.86 76.33) (end 180.304315 76.33) (width 0.2) (layer "F.Cu") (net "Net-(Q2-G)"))
 (segment (start 180.304315 76.33) (end 181.61 77.635685) (width 0.2) (layer "F.Cu") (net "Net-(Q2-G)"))
 (segment (start 177.8 82.55) (end 178.69 82.55) (width 0.2) (layer "F.Cu") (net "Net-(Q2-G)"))
 (segment (start 178.69 82.55) (end 181.61 79.63) (width 0.2) (layer "F.Cu") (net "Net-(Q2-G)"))
 (segment (start 177.8 81.2925) (end 177.4675 80.96) (width 0.2) (layer "F.Cu") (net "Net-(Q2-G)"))
 (segment (start 166.37 82.55) (end 167.64 82.55) (width 0.2) (layer "F.Cu") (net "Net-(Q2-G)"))
 (segment (start 177.8 82.55) (end 177.8 81.2925) (width 0.2) (layer "F.Cu") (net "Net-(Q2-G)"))
 (segment (start 181.61 77.635685) (end 181.61 79.63) (width 0.2) (layer "F.Cu") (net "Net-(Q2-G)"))
 (segment (start 173.99 80.01) (end 172.72 81.28) (width 0.2) (layer "F.Cu") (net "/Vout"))
 (segment (start 175.5925 80.01) (end 173.99 80.01) (width 0.2) (layer "F.Cu") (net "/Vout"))
 (segment (start 187.515 88.425) (end 188.33 87.61) (width 0.2) (layer "F.Cu") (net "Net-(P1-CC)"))
 (segment (start 187.515 88.9) (end 187.515 88.425) (width 0.2) (layer "F.Cu") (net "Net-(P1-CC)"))
 (segment (start 188.33 87.61) (end 189.36 87.61) (width 0.2) (layer "F.Cu") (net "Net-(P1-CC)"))
 (segment (start 173.99 87.25) (end 172.34 88.9) (width 0.2) (layer "F.Cu") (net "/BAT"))
 (segment (start 173.99 86.36) (end 173.99 87.25) (width 0.2) (layer "F.Cu") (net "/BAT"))
 (segment (start 175.26 87.63) (end 173.99 86.36) (width 0.2) (layer "F.Cu") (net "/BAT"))
 (segment (start 180.88 87.63) (end 175.26 87.63) (width 0.2) (layer "F.Cu") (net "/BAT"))
 (segment (start 138.25 85.12) (end 138.25 88.858478) (width 0.2) (layer "F.Cu") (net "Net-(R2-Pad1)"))
 (segment (start 138.25 88.858478) (end 140.831522 91.44) (width 0.2) (layer "F.Cu") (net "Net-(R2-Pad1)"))
 (segment (start 139.55 83.82) (end 146.05 83.82) (width 0.2) (layer "F.Cu") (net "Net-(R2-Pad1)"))
 (segment (start 139.55 83.82) (end 138.25 85.12) (width 0.2) (layer "F.Cu") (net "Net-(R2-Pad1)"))
 (segment (start 140.831522 91.44) (end 144.4 91.44) (width 0.2) (layer "F.Cu") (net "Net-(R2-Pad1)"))
 (segment (start 158.75 83.82) (end 152.25 83.82) (width 0.2) (layer "F.Cu") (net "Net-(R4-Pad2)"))
 (segment (start 158.75 83.82) (end 160.02 82.55) (width 0.2) (layer "F.Cu") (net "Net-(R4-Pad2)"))
 (segment (start 160.02 82.55) (end 164.72 82.55) (width 0.2) (layer "F.Cu") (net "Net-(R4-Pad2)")))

